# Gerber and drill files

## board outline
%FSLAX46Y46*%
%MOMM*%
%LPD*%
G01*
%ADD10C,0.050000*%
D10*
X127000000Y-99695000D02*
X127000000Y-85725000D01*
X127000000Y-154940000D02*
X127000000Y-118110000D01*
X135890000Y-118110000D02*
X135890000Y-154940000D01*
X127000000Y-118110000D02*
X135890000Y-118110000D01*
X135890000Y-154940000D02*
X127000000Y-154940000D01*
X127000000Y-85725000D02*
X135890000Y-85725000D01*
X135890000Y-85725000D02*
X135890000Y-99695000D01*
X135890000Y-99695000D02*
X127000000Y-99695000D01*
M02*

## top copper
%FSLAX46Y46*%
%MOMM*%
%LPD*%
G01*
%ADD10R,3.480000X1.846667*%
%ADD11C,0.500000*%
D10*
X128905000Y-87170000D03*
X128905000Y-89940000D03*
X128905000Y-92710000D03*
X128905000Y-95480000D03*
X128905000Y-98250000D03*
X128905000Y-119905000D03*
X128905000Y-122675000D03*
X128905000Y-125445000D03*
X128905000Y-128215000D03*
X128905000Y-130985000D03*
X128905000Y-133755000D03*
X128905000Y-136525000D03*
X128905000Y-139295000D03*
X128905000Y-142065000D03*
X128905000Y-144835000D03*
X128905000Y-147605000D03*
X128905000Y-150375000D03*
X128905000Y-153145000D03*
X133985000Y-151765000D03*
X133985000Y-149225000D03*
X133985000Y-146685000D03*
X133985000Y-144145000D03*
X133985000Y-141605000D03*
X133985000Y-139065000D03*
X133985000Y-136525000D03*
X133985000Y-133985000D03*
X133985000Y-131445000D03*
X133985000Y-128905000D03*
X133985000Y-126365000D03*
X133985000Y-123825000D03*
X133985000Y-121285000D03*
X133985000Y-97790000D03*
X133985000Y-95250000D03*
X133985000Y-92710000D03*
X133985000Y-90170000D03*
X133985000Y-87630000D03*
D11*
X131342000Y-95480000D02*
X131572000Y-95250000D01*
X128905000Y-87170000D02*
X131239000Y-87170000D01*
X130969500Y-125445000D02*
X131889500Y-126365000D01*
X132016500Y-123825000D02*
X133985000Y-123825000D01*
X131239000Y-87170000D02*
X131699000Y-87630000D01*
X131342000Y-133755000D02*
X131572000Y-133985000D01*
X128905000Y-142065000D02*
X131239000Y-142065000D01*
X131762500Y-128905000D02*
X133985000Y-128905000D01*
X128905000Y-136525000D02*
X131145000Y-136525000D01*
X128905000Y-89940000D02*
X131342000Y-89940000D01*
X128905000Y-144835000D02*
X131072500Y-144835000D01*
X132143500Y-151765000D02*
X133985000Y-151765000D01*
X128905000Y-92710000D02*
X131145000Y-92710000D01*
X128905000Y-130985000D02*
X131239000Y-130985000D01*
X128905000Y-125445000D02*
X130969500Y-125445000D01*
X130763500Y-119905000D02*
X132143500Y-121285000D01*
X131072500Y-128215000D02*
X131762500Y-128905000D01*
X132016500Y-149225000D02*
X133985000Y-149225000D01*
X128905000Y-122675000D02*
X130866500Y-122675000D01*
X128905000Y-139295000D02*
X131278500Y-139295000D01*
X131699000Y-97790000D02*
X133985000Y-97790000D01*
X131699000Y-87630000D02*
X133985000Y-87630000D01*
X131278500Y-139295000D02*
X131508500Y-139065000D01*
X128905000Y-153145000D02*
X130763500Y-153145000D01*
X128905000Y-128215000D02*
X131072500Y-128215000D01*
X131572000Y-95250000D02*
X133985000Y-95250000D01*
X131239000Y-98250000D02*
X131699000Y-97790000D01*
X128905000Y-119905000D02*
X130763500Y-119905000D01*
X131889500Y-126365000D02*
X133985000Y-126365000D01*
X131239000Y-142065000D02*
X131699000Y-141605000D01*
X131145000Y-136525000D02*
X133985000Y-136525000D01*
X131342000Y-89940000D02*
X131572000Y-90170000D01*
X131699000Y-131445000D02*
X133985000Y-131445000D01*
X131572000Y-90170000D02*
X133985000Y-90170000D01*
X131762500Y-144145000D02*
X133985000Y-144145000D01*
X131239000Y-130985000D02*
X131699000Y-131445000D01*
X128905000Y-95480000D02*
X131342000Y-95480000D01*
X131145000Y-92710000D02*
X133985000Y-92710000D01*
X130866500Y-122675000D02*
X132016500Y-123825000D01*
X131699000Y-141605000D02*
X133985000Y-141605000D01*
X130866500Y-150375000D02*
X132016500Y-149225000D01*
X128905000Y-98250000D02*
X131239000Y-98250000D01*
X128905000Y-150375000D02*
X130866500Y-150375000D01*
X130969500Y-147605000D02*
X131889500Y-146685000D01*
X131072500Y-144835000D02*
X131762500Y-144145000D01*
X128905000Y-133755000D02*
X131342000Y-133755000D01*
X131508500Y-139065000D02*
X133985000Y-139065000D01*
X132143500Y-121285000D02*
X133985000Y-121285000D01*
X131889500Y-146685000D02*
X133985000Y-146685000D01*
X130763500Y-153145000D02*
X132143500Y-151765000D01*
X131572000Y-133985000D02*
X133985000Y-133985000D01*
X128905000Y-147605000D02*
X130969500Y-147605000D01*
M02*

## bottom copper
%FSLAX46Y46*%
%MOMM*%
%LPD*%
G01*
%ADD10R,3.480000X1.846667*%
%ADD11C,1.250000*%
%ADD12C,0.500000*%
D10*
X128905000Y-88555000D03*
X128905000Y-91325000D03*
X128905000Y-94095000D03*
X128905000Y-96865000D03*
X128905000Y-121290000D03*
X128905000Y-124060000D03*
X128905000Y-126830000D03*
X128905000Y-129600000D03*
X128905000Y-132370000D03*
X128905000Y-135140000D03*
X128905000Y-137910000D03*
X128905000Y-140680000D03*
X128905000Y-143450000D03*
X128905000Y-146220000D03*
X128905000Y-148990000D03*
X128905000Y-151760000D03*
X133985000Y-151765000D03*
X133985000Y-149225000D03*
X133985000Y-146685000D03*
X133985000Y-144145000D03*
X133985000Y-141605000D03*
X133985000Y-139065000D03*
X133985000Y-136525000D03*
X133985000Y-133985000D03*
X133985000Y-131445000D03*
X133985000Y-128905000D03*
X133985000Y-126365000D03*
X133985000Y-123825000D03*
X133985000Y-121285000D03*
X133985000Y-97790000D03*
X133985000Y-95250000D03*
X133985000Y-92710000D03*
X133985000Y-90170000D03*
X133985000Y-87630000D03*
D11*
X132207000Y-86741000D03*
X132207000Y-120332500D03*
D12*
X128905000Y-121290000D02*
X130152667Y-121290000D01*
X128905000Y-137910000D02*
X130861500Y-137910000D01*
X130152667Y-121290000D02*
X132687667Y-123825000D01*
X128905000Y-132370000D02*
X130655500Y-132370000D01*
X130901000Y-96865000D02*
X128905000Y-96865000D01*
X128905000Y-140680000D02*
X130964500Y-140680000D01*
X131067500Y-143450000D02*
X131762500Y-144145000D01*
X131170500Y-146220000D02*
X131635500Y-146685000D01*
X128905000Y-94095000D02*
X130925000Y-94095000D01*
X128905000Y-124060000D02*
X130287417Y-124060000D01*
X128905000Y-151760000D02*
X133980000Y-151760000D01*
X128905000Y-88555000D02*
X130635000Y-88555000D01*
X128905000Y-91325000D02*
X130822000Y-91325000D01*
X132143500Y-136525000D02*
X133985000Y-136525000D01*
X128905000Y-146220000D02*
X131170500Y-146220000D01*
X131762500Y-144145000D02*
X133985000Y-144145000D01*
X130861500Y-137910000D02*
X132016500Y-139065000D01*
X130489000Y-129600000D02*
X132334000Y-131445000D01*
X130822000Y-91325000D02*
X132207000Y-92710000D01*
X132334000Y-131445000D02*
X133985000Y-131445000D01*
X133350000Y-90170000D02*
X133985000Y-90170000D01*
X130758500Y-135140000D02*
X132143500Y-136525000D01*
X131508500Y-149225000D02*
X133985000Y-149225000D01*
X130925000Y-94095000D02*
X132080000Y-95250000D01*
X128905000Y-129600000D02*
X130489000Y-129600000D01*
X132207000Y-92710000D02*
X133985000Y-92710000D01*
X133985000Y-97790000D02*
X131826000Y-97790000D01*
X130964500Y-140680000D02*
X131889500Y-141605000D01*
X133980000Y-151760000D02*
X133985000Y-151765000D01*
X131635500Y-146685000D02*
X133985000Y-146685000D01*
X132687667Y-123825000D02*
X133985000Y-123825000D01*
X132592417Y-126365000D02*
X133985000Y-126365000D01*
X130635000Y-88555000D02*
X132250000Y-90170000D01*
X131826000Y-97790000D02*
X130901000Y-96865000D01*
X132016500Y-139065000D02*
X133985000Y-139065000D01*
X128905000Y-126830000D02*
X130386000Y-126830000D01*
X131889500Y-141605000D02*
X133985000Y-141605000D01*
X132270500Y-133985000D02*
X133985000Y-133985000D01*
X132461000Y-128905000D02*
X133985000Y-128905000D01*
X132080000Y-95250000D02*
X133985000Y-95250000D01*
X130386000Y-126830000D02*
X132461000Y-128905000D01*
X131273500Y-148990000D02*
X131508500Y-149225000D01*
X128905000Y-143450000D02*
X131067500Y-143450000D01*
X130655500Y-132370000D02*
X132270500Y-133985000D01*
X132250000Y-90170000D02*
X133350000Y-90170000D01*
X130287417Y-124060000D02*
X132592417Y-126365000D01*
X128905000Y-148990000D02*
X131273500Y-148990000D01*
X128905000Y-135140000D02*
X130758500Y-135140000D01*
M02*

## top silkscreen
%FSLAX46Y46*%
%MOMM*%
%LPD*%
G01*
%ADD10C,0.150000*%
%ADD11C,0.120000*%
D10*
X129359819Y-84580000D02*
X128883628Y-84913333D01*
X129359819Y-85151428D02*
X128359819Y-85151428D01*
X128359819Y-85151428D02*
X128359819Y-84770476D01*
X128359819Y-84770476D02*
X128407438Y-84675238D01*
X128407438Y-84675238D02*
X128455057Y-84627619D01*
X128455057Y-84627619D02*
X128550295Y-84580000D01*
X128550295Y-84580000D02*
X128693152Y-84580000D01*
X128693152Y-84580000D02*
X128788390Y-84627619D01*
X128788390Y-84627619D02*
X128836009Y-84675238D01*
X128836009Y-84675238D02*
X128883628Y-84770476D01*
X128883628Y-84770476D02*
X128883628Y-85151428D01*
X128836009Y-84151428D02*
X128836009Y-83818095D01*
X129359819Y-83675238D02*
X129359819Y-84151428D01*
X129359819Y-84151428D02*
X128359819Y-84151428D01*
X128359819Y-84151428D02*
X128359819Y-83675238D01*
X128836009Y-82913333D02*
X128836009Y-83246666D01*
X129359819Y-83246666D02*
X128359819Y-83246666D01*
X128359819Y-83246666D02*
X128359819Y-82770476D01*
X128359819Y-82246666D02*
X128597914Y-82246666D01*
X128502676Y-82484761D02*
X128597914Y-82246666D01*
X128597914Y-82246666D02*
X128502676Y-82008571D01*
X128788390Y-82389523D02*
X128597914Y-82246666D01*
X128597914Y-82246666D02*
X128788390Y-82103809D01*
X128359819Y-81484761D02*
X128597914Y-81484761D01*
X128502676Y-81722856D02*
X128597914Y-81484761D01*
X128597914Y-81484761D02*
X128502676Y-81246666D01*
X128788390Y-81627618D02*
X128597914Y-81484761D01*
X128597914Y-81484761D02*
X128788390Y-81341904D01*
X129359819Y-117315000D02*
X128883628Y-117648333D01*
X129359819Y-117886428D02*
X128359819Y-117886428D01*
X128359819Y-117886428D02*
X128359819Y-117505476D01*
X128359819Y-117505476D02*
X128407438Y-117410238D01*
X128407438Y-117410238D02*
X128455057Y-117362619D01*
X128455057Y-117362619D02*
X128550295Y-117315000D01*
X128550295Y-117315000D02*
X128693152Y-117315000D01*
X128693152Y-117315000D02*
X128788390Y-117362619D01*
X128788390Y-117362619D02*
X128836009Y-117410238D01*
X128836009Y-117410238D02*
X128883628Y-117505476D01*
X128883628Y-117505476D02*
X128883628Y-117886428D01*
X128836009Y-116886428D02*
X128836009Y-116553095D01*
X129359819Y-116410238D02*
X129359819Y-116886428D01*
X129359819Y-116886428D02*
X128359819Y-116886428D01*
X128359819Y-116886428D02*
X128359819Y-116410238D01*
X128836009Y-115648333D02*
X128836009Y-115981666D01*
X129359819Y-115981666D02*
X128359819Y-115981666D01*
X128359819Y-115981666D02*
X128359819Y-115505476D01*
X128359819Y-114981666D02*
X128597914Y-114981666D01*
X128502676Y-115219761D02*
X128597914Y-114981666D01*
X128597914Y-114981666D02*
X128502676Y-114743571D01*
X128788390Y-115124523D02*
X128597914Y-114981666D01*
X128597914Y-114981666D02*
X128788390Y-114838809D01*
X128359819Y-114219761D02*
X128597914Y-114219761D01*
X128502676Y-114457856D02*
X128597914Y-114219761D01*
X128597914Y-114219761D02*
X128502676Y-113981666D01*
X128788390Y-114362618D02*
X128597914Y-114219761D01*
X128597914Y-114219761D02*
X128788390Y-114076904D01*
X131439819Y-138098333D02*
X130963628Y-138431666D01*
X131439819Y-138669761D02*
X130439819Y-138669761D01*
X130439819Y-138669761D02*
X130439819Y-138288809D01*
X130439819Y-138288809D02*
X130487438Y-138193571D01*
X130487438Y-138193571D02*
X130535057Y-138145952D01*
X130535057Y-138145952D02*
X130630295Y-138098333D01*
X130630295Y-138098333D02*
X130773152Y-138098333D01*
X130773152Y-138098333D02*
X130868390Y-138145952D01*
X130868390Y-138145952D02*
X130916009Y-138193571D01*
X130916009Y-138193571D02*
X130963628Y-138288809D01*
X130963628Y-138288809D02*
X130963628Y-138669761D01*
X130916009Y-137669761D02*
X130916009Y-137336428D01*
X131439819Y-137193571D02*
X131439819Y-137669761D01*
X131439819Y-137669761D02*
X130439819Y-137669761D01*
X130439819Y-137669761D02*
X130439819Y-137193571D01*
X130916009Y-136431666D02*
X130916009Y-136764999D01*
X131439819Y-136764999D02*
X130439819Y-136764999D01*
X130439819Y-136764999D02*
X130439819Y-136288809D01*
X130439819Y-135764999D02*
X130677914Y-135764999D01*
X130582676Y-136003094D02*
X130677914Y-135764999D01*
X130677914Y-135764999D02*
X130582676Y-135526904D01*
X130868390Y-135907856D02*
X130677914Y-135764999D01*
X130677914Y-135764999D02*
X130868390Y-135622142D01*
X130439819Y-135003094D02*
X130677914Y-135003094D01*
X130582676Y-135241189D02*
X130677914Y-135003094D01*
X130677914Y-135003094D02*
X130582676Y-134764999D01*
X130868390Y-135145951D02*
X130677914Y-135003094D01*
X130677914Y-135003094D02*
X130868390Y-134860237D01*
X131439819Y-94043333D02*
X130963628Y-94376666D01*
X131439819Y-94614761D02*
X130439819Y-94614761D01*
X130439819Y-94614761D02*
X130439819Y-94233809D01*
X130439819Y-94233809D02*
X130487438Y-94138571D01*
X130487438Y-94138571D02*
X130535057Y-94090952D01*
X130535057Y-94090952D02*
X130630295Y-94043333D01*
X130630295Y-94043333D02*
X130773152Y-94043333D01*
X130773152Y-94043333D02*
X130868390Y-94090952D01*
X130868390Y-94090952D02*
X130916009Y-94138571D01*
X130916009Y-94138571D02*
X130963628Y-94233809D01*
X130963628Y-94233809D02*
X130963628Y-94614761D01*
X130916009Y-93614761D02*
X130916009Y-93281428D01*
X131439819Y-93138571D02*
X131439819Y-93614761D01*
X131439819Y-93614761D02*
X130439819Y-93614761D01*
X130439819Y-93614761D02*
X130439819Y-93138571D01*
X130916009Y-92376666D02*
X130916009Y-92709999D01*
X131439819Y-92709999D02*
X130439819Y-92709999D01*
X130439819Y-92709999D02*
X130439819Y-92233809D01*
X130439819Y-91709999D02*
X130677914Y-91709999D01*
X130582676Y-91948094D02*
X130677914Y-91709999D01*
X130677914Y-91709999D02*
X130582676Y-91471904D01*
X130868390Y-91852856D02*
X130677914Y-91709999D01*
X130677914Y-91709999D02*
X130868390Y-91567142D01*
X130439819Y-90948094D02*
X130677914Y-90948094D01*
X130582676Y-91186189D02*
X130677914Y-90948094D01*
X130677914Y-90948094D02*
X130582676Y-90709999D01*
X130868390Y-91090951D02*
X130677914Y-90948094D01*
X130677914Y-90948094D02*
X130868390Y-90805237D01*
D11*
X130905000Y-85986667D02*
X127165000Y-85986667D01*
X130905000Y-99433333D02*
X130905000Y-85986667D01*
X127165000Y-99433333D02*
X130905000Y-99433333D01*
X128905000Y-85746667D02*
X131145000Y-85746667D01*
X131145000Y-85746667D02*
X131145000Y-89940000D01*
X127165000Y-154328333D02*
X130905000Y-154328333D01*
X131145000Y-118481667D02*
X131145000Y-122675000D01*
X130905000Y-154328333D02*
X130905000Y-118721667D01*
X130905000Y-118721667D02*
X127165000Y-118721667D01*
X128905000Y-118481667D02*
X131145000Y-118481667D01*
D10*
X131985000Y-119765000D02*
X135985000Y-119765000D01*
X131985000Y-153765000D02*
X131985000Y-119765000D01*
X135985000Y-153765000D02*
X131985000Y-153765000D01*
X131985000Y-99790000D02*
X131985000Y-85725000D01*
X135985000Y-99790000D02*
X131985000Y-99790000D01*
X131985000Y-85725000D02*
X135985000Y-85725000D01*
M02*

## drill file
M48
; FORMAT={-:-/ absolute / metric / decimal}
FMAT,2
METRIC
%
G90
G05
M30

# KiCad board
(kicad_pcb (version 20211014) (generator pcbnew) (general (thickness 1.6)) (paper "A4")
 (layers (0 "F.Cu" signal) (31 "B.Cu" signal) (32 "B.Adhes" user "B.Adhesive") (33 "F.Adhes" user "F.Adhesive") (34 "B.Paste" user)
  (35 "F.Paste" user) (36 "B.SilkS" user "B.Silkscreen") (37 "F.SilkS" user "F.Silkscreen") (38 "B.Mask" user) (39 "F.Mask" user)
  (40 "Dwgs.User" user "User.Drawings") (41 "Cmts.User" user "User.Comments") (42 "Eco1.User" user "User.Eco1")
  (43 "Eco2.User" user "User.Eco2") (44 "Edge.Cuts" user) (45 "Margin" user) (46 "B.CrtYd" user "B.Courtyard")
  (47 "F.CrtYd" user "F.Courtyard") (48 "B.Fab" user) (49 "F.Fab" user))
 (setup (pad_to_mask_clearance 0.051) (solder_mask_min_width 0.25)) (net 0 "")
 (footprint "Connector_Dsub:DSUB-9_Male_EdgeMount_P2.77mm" (layer "F.Cu") (at 128.905 92.71 -90)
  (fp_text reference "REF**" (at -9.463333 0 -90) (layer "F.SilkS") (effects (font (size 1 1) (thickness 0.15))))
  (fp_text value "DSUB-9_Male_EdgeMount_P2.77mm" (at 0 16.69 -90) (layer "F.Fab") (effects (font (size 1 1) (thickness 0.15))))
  (fp_line (start -6.723333 -2) (end -6.723333 1.74) (layer "F.SilkS") (width 0.12))
  (fp_line (start 6.723333 -2) (end -6.723333 -2) (layer "F.SilkS") (width 0.12))
  (fp_line (start 6.723333 1.74) (end 6.723333 -2) (layer "F.SilkS") (width 0.12))
  (fp_line (start -6.963333 0) (end -6.963333 -2.24) (layer "F.SilkS") (width 0.12))
  (fp_line (start -6.963333 -2.24) (end -2.77 -2.24) (layer "F.SilkS") (width 0.12))
  (pad "1" smd rect (at -5.54 0 270) (size 1.846667 3.48) (layers "F.Cu" "F.Paste" "F.Mask"))
  (pad "2" smd rect (at -2.77 0 270) (size 1.846667 3.48) (layers "F.Cu" "F.Paste" "F.Mask"))
  (pad "3" smd rect (at 0 0 270) (size 1.846667 3.48) (layers "F.Cu" "F.Paste" "F.Mask"))
  (pad "4" smd rect (at 2.77 0 270) (size 1.846667 3.48) (layers "F.Cu" "F.Paste" "F.Mask"))
  (pad "5" smd rect (at 5.54 0 270) (size 1.846667 3.48) (layers "F.Cu" "F.Paste" "F.Mask"))
  (pad "6" smd rect (at -4.155 0 270) (size 1.846667 3.48) (layers "B.Cu" "B.Paste" "B.Mask"))
  (pad "7" smd rect (at -1.385 0 270) (size 1.846667 3.48) (layers "B.Cu" "B.Paste" "B.Mask"))
  (pad "8" smd rect (at 1.385 0 270) (size 1.846667 3.48) (layers "B.Cu" "B.Paste" "B.Mask"))
  (pad "9" smd rect (at 4.155 0 270) (size 1.846667 3.48) (layers "B.Cu" "B.Paste" "B.Mask")))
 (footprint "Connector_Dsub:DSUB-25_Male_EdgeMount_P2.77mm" (layer "F.Cu") (at 128.905 136.525 -90)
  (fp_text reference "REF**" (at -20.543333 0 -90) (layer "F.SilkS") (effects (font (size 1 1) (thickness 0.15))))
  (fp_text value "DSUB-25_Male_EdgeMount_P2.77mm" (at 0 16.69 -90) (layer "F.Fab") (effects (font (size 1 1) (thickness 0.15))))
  (fp_line (start 17.803333 1.74) (end 17.803333 -2) (layer "F.SilkS") (width 0.12))
  (fp_line (start -18.043333 -2.24) (end -13.85 -2.24) (layer "F.SilkS") (width 0.12))
  (fp_line (start 17.803333 -2) (end -17.803333 -2) (layer "F.SilkS") (width 0.12))
  (fp_line (start -17.803333 -2) (end -17.803333 1.74) (layer "F.SilkS") (width 0.12))
  (fp_line (start -18.043333 0) (end -18.043333 -2.24) (layer "F.SilkS") (width 0.12))
  (pad "1" smd rect (at -16.62 0 270) (size 1.846667 3.48) (layers "F.Cu" "F.Paste" "F.Mask"))
  (pad "2" smd rect (at -13.85 0 270) (size 1.846667 3.48) (layers "F.Cu" "F.Paste" "F.Mask"))
  (pad "3" smd rect (at -11.08 0 270) (size 1.846667 3.48) (layers "F.Cu" "F.Paste" "F.Mask"))
  (pad "4" smd rect (at -8.31 0 270) (size 1.846667 3.48) (layers "F.Cu" "F.Paste" "F.Mask"))
  (pad "5" smd rect (at -5.54 0 270) (size 1.846667 3.48) (layers "F.Cu" "F.Paste" "F.Mask"))
  (pad "6" smd rect (at -2.77 0 270) (size 1.846667 3.48) (layers "F.Cu" "F.Paste" "F.Mask"))
  (pad "7" smd rect (at 0 0 270) (size 1.846667 3.48) (layers "F.Cu" "F.Paste" "F.Mask"))
  (pad "8" smd rect (at 2.77 0 270) (size 1.846667 3.48) (layers "F.Cu" "F.Paste" "F.Mask"))
  (pad "9" smd rect (at 5.54 0 270) (size 1.846667 3.48) (layers "F.Cu" "F.Paste" "F.Mask"))
  (pad "10" smd rect (at 8.31 0 270) (size 1.846667 3.48) (layers "F.Cu" "F.Paste" "F.Mask"))
  (pad "11" smd rect (at 11.08 0 270) (size 1.846667 3.48) (layers "F.Cu" "F.Paste" "F.Mask"))
  (pad "12" smd rect (at 13.85 0 270) (size 1.846667 3.48) (layers "F.Cu" "F.Paste" "F.Mask"))
  (pad "13" smd rect (at 16.62 0 270) (size 1.846667 3.48) (layers "F.Cu" "F.Paste" "F.Mask"))
  (pad "14" smd rect (at -15.235 0 270) (size 1.846667 3.48) (layers "B.Cu" "B.Paste" "B.Mask"))
  (pad "15" smd rect (at -12.465 0 270) (size 1.846667 3.48) (layers "B.Cu" "B.Paste" "B.Mask"))
  (pad "16" smd rect (at -9.695 0 270) (size 1.846667 3.48) (layers "B.Cu" "B.Paste" "B.Mask"))
  (pad "17" smd rect (at -6.925 0 270) (size 1.846667 3.48) (layers "B.Cu" "B.Paste" "B.Mask"))
  (pad "18" smd rect (at -4.155 0 270) (size 1.846667 3.48) (layers "B.Cu" "B.Paste" "B.Mask"))
  (pad "19" smd rect (at -1.385 0 270) (size 1.846667 3.48) (layers "B.Cu" "B.Paste" "B.Mask"))
  (pad "20" smd rect (at 1.385 0 270) (size 1.846667 3.48) (layers "B.Cu" "B.Paste" "B.Mask"))
  (pad "21" smd rect (at 4.155 0 270) (size 1.846667 3.48) (layers "B.Cu" "B.Paste" "B.Mask"))
  (pad "22" smd rect (at 6.925 0 270) (size 1.846667 3.48) (layers "B.Cu" "B.Paste" "B.Mask"))
  (pad "23" smd rect (at 9.695 0 270) (size 1.846667 3.48) (layers "B.Cu" "B.Paste" "B.Mask"))
  (pad "24" smd rect (at 12.465 0 270) (size 1.846667 3.48) (layers "B.Cu" "B.Paste" "B.Mask"))
  (pad "25" smd rect (at 15.235 0 270) (size 1.846667 3.48) (layers "B.Cu" "B.Paste" "B.Mask")))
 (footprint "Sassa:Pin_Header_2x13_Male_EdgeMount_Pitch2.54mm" (layer "F.Cu") (at 133.985 151.765 90)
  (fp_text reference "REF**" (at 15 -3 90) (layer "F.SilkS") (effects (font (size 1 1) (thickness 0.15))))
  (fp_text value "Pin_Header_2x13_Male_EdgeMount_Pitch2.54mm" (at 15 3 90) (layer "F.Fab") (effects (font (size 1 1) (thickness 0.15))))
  (fp_line (start 32 -2) (end 32 2) (layer "F.SilkS") (width 0.15))
  (fp_line (start -2 -2) (end 32 -2) (layer "F.SilkS") (width 0.15))
  (fp_line (start -2 2) (end -2 -2) (layer "F.SilkS") (width 0.15))
  (pad "1" smd rect locked (at 0 0 90) (size 1.846667 3.48) (layers "B.Cu" "B.Paste" "B.Mask"))
  (pad "2" smd rect locked (at 0 0 90) (size 1.846667 3.48) (layers "F.Cu" "F.Paste" "F.Mask"))
  (pad "3" smd rect locked (at 2.54 0 90) (size 1.846667 3.48) (layers "B.Cu" "B.Paste" "B.Mask"))
  (pad "4" smd rect locked (at 2.54 0 90) (size 1.846667 3.48) (layers "F.Cu" "F.Paste" "F.Mask"))
  (pad "5" smd rect locked (at 5.08 0 90) (size 1.846667 3.48) (layers "B.Cu" "B.Paste" "B.Mask"))
  (pad "6" smd rect locked (at 5.08 0 90) (size 1.846667 3.48) (layers "F.Cu" "F.Paste" "F.Mask"))
  (pad "7" smd rect locked (at 7.62 0 90) (size 1.846667 3.48) (layers "B.Cu" "B.Paste" "B.Mask"))
  (pad "8" smd rect locked (at 7.62 0 90) (size 1.846667 3.48) (layers "F.Cu" "F.Paste" "F.Mask"))
  (pad "9" smd rect locked (at 10.16 0 90) (size 1.846667 3.48) (layers "B.Cu" "B.Paste" "B.Mask"))
  (pad "10" smd rect locked (at 10.16 0 90) (size 1.846667 3.48) (layers "F.Cu" "F.Paste" "F.Mask"))
  (pad "11" smd rect locked (at 12.7 0 90) (size 1.846667 3.48) (layers "B.Cu" "B.Paste" "B.Mask"))
  (pad "12" smd rect locked (at 12.7 0 90) (size 1.846667 3.48) (layers "F.Cu" "F.Paste" "F.Mask"))
  (pad "13" smd rect locked (at 15.24 0 90) (size 1.846667 3.48) (layers "B.Cu" "B.Paste" "B.Mask"))
  (pad "14" smd rect locked (at 15.24 0 90) (size 1.846667 3.48) (layers "F.Cu" "F.Paste" "F.Mask"))
  (pad "15" smd rect locked (at 17.78 0 90) (size 1.846667 3.48) (layers "B.Cu" "B.Paste" "B.Mask"))
  (pad "16" smd rect locked (at 17.78 0 90) (size 1.846667 3.48) (layers "F.Cu" "F.Paste" "F.Mask"))
  (pad "17" smd rect locked (at 20.32 0 90) (size 1.846667 3.48) (layers "B.Cu" "B.Paste" "B.Mask"))
  (pad "18" smd rect locked (at 20.32 0 90) (size 1.846667 3.48) (layers "F.Cu" "F.Paste" "F.Mask"))
  (pad "19" smd rect locked (at 22.86 0 90) (size 1.846667 3.48) (layers "B.Cu" "B.Paste" "B.Mask"))
  (pad "20" smd rect locked (at 22.86 0 90) (size 1.846667 3.48) (layers "F.Cu" "F.Paste" "F.Mask"))
  (pad "21" smd rect locked (at 25.4 0 90) (size 1.846667 3.48) (layers "B.Cu" "B.Paste" "B.Mask"))
  (pad "22" smd rect locked (at 25.4 0 90) (size 1.846667 3.48) (layers "F.Cu" "F.Paste" "F.Mask"))
  (pad "23" smd rect locked (at 27.94 0 90) (size 1.846667 3.48) (layers "B.Cu" "B.Paste" "B.Mask"))
  (pad "24" smd rect locked (at 27.94 0 90) (size 1.846667 3.48) (layers "F.Cu" "F.Paste" "F.Mask"))
  (pad "25" smd rect locked (at 30.48 0 90) (size 1.846667 3.48) (layers "B.Cu" "B.Paste" "B.Mask"))
  (pad "26" smd rect locked (at 30.48 0 90) (size 1.846667 3.48) (layers "F.Cu" "F.Paste" "F.Mask")))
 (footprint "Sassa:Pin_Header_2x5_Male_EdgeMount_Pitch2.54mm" (layer "F.Cu") (at 133.985 97.79 90)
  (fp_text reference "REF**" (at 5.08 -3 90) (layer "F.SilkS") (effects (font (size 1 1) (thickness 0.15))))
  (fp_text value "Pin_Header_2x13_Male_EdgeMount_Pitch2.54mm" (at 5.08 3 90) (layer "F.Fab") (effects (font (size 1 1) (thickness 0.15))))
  (fp_line (start -2 -2) (end 12.065 -2) (layer "F.SilkS") (width 0.15))
  (fp_line (start -2 2) (end -2 -2) (layer "F.SilkS") (width 0.15))
  (fp_line (start 12.065 -2) (end 12.065 2) (layer "F.SilkS") (width 0.15))
  (pad "1" smd rect locked (at 0 0 90) (size 1.846667 3.48) (layers "B.Cu" "B.Paste" "B.Mask"))
  (pad "2" smd rect locked (at 0 0 90) (size 1.846667 3.48) (layers "F.Cu" "F.Paste" "F.Mask"))
  (pad "3" smd rect locked (at 2.54 0 90) (size 1.846667 3.48) (layers "B.Cu" "B.Paste" "B.Mask"))
  (pad "4" smd rect locked (at 2.54 0 90) (size 1.846667 3.48) (layers "F.Cu" "F.Paste" "F.Mask"))
  (pad "5" smd rect locked (at 5.08 0 90) (size 1.846667 3.48) (layers "B.Cu" "B.Paste" "B.Mask"))
  (pad "6" smd rect locked (at 5.08 0 90) (size 1.846667 3.48) (layers "F.Cu" "F.Paste" "F.Mask"))
  (pad "7" smd rect locked (at 7.62 0 90) (size 1.846667 3.48) (layers "B.Cu" "B.Paste" "B.Mask"))
  (pad "8" smd rect locked (at 7.62 0 90) (size 1.846667 3.48) (layers "F.Cu" "F.Paste" "F.Mask"))
  (pad "9" smd rect locked (at 10.16 0 90) (size 1.846667 3.48) (layers "B.Cu" "B.Paste" "B.Mask"))
  (pad "10" smd rect locked (at 10.16 0 90) (size 1.846667 3.48) (layers "F.Cu" "F.Paste" "F.Mask")))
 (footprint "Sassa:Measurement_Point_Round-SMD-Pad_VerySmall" (layer "B.Cu") (at 132.207 86.741)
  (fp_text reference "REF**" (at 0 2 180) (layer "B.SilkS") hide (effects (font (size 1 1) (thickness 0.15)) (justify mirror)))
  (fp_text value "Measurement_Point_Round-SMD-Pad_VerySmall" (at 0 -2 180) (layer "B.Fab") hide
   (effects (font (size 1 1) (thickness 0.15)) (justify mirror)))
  (pad "1" smd circle locked (at 0 0) (size 1.25 1.25) (layers "B.Cu" "B.Mask")))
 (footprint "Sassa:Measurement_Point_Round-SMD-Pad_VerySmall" (layer "B.Cu") (at 132.207 120.3325)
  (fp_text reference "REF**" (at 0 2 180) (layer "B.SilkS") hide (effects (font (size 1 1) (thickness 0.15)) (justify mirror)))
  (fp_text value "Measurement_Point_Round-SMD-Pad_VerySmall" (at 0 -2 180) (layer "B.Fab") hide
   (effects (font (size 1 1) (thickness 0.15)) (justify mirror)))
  (pad "1" smd circle locked (at 0 0) (size 1.25 1.25) (layers "B.Cu" "B.Mask")))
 (gr_line (start 127 99.695) (end 127 85.725) (layer "Edge.Cuts") (width 0.05))
 (gr_line (start 127 154.94) (end 127 118.11) (layer "Edge.Cuts") (width 0.05))
 (gr_line (start 135.89 118.11) (end 135.89 154.94) (layer "Edge.Cuts") (width 0.05))
 (gr_line (start 127 118.11) (end 135.89 118.11) (layer "Edge.Cuts") (width 0.05))
 (gr_line (start 135.89 154.94) (end 127 154.94) (layer "Edge.Cuts") (width 0.05))
 (gr_line (start 127 85.725) (end 135.89 85.725) (layer "Edge.Cuts") (width 0.05))
 (gr_line (start 135.89 85.725) (end 135.89 99.695) (layer "Edge.Cuts") (width 0.05))
 (gr_line (start 135.89 99.695) (end 127 99.695) (layer "Edge.Cuts") (width 0.05))
 (segment (start 131.342 95.48) (end 131.572 95.25) (width 0.5) (layer "F.Cu") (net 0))
 (segment (start 128.905 87.17) (end 131.239 87.17) (width 0.5) (layer "F.Cu") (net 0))
 (segment (start 130.9695 125.445) (end 131.8895 126.365) (width 0.5) (layer "F.Cu") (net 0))
 (segment (start 132.0165 123.825) (end 133.985 123.825) (width 0.5) (layer "F.Cu") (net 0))
 (segment (start 131.239 87.17) (end 131.699 87.63) (width 0.5) (layer "F.Cu") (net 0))
 (segment (start 131.342 133.755) (end 131.572 133.985) (width 0.5) (layer "F.Cu") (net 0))
 (segment (start 128.905 142.065) (end 131.239 142.065) (width 0.5) (layer "F.Cu") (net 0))
 (segment (start 131.7625 128.905) (end 133.985 128.905) (width 0.5) (layer "F.Cu") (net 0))
 (segment (start 128.905 136.525) (end 131.145 136.525) (width 0.5) (layer "F.Cu") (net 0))
 (segment (start 128.905 89.94) (end 131.342 89.94) (width 0.5) (layer "F.Cu") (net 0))
 (segment (start 128.905 144.835) (end 131.0725 144.835) (width 0.5) (layer "F.Cu") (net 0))
 (segment (start 132.1435 151.765) (end 133.985 151.765) (width 0.5) (layer "F.Cu") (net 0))
 (segment (start 128.905 92.71) (end 131.145 92.71) (width 0.5) (layer "F.Cu") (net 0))
 (segment (start 128.905 130.985) (end 131.239 130.985) (width 0.5) (layer "F.Cu") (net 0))
 (segment (start 128.905 125.445) (end 130.9695 125.445) (width 0.5) (layer "F.Cu") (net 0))
 (segment (start 130.7635 119.905) (end 132.1435 121.285) (width 0.5) (layer "F.Cu") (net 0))
 (segment (start 131.0725 128.215) (end 131.7625 128.905) (width 0.5) (layer "F.Cu") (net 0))
 (segment (start 132.0165 149.225) (end 133.985 149.225) (width 0.5) (layer "F.Cu") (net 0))
 (segment (start 128.905 122.675) (end 130.8665 122.675) (width 0.5) (layer "F.Cu") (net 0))
 (segment (start 128.905 139.295) (end 131.2785 139.295) (width 0.5) (layer "F.Cu") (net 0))
 (segment (start 131.699 97.79) (end 133.985 97.79) (width 0.5) (layer "F.Cu") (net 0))
 (segment (start 131.699 87.63) (end 133.985 87.63) (width 0.5) (layer "F.Cu") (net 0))
 (segment (start 131.2785 139.295) (end 131.5085 139.065) (width 0.5) (layer "F.Cu") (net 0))
 (segment (start 128.905 153.145) (end 130.7635 153.145) (width 0.5) (layer "F.Cu") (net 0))
 (segment (start 128.905 128.215) (end 131.0725 128.215) (width 0.5) (layer "F.Cu") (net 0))
 (segment (start 131.572 95.25) (end 133.985 95.25) (width 0.5) (layer "F.Cu") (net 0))
 (segment (start 131.239 98.25) (end 131.699 97.79) (width 0.5) (layer "F.Cu") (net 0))
 (segment (start 128.905 119.905) (end 130.7635 119.905) (width 0.5) (layer "F.Cu") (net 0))
 (segment (start 131.8895 126.365) (end 133.985 126.365) (width 0.5) (layer "F.Cu") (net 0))
 (segment (start 131.239 142.065) (end 131.699 141.605) (width 0.5) (layer "F.Cu") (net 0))
 (segment (start 131.145 136.525) (end 133.985 136.525) (width 0.5) (layer "F.Cu") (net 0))
 (segment (start 131.342 89.94) (end 131.572 90.17) (width 0.5) (layer "F.Cu") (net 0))
 (segment (start 131.699 131.445) (end 133.985 131.445) (width 0.5) (layer "F.Cu") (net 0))
 (segment (start 131.572 90.17) (end 133.985 90.17) (width 0.5) (layer "F.Cu") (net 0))
 (segment (start 131.7625 144.145) (end 133.985 144.145) (width 0.5) (layer "F.Cu") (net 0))
 (segment (start 131.239 130.985) (end 131.699 131.445) (width 0.5) (layer "F.Cu") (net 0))
 (segment (start 128.905 95.48) (end 131.342 95.48) (width 0.5) (layer "F.Cu") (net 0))
 (segment (start 131.145 92.71) (end 133.985 92.71) (width 0.5) (layer "F.Cu") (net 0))
 (segment (start 130.8665 122.675) (end 132.0165 123.825) (width 0.5) (layer "F.Cu") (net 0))
 (segment (start 131.699 141.605) (end 133.985 141.605) (width 0.5) (layer "F.Cu") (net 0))
 (segment (start 130.8665 150.375) (end 132.0165 149.225) (width 0.5) (layer "F.Cu") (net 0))
 (segment (start 128.905 98.25) (end 131.239 98.25) (width 0.5) (layer "F.Cu") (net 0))
 (segment (start 128.905 150.375) (end 130.8665 150.375) (width 0.5) (layer "F.Cu") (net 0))
 (segment (start 130.9695 147.605) (end 131.8895 146.685) (width 0.5) (layer "F.Cu") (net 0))
 (segment (start 131.0725 144.835) (end 131.7625 144.145) (width 0.5) (layer "F.Cu") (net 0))
 (segment (start 128.905 133.755) (end 131.342 133.755) (width 0.5) (layer "F.Cu") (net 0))
 (segment (start 131.5085 139.065) (end 133.985 139.065) (width 0.5) (layer "F.Cu") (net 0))
 (segment (start 132.1435 121.285) (end 133.985 121.285) (width 0.5) (layer "F.Cu") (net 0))
 (segment (start 131.8895 146.685) (end 133.985 146.685) (width 0.5) (layer "F.Cu") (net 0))
 (segment (start 130.7635 153.145) (end 132.1435 151.765) (width 0.5) (layer "F.Cu") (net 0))
 (segment (start 131.572 133.985) (end 133.985 133.985) (width 0.5) (layer "F.Cu") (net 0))
 (segment (start 128.905 147.605) (end 130.9695 147.605) (width 0.5) (layer "F.Cu") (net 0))
 (segment (start 128.905 121.29) (end 130.152667 121.29) (width 0.5) (layer "B.Cu") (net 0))
 (segment (start 128.905 137.91) (end 130.8615 137.91) (width 0.5) (layer "B.Cu") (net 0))
 (segment (start 130.152667 121.29) (end 132.687667 123.825) (width 0.5) (layer "B.Cu") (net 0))
 (segment (start 128.905 132.37) (end 130.6555 132.37) (width 0.5) (layer "B.Cu") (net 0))
 (segment (start 130.901 96.865) (end 128.905 96.865) (width 0.5) (layer "B.Cu") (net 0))
 (segment (start 128.905 140.68) (end 130.9645 140.68) (width 0.5) (layer "B.Cu") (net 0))
 (segment (start 131.0675 143.45) (end 131.7625 144.145) (width 0.5) (layer "B.Cu") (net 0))
 (segment (start 131.1705 146.22) (end 131.6355 146.685) (width 0.5) (layer "B.Cu") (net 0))
 (segment (start 128.905 94.095) (end 130.925 94.095) (width 0.5) (layer "B.Cu") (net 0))
 (segment (start 128.905 124.06) (end 130.287417 124.06) (width 0.5) (layer "B.Cu") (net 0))
 (segment (start 128.905 151.76) (end 133.98 151.76) (width 0.5) (layer "B.Cu") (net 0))
 (segment (start 128.905 88.555) (end 130.635 88.555) (width 0.5) (layer "B.Cu") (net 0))
 (segment (start 128.905 91.325) (end 130.822 91.325) (width 0.5) (layer "B.Cu") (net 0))
 (segment (start 132.1435 136.525) (end 133.985 136.525) (width 0.5) (layer "B.Cu") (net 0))
 (segment (start 128.905 146.22) (end 131.1705 146.22) (width 0.5) (layer "B.Cu") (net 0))
 (segment (start 131.7625 144.145) (end 133.985 144.145) (width 0.5) (layer "B.Cu") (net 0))
 (segment (start 130.8615 137.91) (end 132.0165 139.065) (width 0.5) (layer "B.Cu") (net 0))
 (segment (start 130.489 129.6) (end 132.334 131.445) (width 0.5) (layer "B.Cu") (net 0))
 (segment (start 130.822 91.325) (end 132.207 92.71) (width 0.5) (layer "B.Cu") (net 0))
 (segment (start 132.334 131.445) (end 133.985 131.445) (width 0.5) (layer "B.Cu") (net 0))
 (segment (start 133.35 90.17) (end 133.985 90.17) (width 0.5) (layer "B.Cu") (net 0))
 (segment (start 130.7585 135.14) (end 132.1435 136.525) (width 0.5) (layer "B.Cu") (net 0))
 (segment (start 131.5085 149.225) (end 133.985 149.225) (width 0.5) (layer "B.Cu") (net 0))
 (segment (start 130.925 94.095) (end 132.08 95.25) (width 0.5) (layer "B.Cu") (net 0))
 (segment (start 128.905 129.6) (end 130.489 129.6) (width 0.5) (layer "B.Cu") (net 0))
 (segment (start 132.207 92.71) (end 133.985 92.71) (width 0.5) (layer "B.Cu") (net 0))
 (segment (start 133.985 97.79) (end 131.826 97.79) (width 0.5) (layer "B.Cu") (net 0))
 (segment (start 130.9645 140.68) (end 131.8895 141.605) (width 0.5) (layer "B.Cu") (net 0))
 (segment (start 133.98 151.76) (end 133.985 151.765) (width 0.5) (layer "B.Cu") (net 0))
 (segment (start 131.6355 146.685) (end 133.985 146.685) (width 0.5) (layer "B.Cu") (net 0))
 (segment (start 132.687667 123.825) (end 133.985 123.825) (width 0.5) (layer "B.Cu") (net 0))
 (segment (start 132.592417 126.365) (end 133.985 126.365) (width 0.5) (layer "B.Cu") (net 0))
 (segment (start 130.635 88.555) (end 132.25 90.17) (width 0.5) (layer "B.Cu") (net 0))
 (segment (start 131.826 97.79) (end 130.901 96.865) (width 0.5) (layer "B.Cu") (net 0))
 (segment (start 132.0165 139.065) (end 133.985 139.065) (width 0.5) (layer "B.Cu") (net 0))
 (segment (start 128.905 126.83) (end 130.386 126.83) (width 0.5) (layer "B.Cu") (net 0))
 (segment (start 131.8895 141.605) (end 133.985 141.605) (width 0.5) (layer "B.Cu") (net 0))
 (segment (start 132.2705 133.985) (end 133.985 133.985) (width 0.5) (layer "B.Cu") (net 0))
 (segment (start 132.461 128.905) (end 133.985 128.905) (width 0.5) (layer "B.Cu") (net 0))
 (segment (start 132.08 95.25) (end 133.985 95.25) (width 0.5) (layer "B.Cu") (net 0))
 (segment (start 130.386 126.83) (end 132.461 128.905) (width 0.5) (layer "B.Cu") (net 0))
 (segment (start 131.2735 148.99) (end 131.5085 149.225) (width 0.5) (layer "B.Cu") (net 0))
 (segment (start 128.905 143.45) (end 131.0675 143.45) (width 0.5) (layer "B.Cu") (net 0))
 (segment (start 130.6555 132.37) (end 132.2705 133.985) (width 0.5) (layer "B.Cu") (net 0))
 (segment (start 132.25 90.17) (end 133.35 90.17) (width 0.5) (layer "B.Cu") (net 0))
 (segment (start 130.287417 124.06) (end 132.592417 126.365) (width 0.5) (layer "B.Cu") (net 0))
 (segment (start 128.905 148.99) (end 131.2735 148.99) (width 0.5) (layer "B.Cu") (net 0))
 (segment (start 128.905 135.14) (end 130.7585 135.14) (width 0.5) (layer "B.Cu") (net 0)))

